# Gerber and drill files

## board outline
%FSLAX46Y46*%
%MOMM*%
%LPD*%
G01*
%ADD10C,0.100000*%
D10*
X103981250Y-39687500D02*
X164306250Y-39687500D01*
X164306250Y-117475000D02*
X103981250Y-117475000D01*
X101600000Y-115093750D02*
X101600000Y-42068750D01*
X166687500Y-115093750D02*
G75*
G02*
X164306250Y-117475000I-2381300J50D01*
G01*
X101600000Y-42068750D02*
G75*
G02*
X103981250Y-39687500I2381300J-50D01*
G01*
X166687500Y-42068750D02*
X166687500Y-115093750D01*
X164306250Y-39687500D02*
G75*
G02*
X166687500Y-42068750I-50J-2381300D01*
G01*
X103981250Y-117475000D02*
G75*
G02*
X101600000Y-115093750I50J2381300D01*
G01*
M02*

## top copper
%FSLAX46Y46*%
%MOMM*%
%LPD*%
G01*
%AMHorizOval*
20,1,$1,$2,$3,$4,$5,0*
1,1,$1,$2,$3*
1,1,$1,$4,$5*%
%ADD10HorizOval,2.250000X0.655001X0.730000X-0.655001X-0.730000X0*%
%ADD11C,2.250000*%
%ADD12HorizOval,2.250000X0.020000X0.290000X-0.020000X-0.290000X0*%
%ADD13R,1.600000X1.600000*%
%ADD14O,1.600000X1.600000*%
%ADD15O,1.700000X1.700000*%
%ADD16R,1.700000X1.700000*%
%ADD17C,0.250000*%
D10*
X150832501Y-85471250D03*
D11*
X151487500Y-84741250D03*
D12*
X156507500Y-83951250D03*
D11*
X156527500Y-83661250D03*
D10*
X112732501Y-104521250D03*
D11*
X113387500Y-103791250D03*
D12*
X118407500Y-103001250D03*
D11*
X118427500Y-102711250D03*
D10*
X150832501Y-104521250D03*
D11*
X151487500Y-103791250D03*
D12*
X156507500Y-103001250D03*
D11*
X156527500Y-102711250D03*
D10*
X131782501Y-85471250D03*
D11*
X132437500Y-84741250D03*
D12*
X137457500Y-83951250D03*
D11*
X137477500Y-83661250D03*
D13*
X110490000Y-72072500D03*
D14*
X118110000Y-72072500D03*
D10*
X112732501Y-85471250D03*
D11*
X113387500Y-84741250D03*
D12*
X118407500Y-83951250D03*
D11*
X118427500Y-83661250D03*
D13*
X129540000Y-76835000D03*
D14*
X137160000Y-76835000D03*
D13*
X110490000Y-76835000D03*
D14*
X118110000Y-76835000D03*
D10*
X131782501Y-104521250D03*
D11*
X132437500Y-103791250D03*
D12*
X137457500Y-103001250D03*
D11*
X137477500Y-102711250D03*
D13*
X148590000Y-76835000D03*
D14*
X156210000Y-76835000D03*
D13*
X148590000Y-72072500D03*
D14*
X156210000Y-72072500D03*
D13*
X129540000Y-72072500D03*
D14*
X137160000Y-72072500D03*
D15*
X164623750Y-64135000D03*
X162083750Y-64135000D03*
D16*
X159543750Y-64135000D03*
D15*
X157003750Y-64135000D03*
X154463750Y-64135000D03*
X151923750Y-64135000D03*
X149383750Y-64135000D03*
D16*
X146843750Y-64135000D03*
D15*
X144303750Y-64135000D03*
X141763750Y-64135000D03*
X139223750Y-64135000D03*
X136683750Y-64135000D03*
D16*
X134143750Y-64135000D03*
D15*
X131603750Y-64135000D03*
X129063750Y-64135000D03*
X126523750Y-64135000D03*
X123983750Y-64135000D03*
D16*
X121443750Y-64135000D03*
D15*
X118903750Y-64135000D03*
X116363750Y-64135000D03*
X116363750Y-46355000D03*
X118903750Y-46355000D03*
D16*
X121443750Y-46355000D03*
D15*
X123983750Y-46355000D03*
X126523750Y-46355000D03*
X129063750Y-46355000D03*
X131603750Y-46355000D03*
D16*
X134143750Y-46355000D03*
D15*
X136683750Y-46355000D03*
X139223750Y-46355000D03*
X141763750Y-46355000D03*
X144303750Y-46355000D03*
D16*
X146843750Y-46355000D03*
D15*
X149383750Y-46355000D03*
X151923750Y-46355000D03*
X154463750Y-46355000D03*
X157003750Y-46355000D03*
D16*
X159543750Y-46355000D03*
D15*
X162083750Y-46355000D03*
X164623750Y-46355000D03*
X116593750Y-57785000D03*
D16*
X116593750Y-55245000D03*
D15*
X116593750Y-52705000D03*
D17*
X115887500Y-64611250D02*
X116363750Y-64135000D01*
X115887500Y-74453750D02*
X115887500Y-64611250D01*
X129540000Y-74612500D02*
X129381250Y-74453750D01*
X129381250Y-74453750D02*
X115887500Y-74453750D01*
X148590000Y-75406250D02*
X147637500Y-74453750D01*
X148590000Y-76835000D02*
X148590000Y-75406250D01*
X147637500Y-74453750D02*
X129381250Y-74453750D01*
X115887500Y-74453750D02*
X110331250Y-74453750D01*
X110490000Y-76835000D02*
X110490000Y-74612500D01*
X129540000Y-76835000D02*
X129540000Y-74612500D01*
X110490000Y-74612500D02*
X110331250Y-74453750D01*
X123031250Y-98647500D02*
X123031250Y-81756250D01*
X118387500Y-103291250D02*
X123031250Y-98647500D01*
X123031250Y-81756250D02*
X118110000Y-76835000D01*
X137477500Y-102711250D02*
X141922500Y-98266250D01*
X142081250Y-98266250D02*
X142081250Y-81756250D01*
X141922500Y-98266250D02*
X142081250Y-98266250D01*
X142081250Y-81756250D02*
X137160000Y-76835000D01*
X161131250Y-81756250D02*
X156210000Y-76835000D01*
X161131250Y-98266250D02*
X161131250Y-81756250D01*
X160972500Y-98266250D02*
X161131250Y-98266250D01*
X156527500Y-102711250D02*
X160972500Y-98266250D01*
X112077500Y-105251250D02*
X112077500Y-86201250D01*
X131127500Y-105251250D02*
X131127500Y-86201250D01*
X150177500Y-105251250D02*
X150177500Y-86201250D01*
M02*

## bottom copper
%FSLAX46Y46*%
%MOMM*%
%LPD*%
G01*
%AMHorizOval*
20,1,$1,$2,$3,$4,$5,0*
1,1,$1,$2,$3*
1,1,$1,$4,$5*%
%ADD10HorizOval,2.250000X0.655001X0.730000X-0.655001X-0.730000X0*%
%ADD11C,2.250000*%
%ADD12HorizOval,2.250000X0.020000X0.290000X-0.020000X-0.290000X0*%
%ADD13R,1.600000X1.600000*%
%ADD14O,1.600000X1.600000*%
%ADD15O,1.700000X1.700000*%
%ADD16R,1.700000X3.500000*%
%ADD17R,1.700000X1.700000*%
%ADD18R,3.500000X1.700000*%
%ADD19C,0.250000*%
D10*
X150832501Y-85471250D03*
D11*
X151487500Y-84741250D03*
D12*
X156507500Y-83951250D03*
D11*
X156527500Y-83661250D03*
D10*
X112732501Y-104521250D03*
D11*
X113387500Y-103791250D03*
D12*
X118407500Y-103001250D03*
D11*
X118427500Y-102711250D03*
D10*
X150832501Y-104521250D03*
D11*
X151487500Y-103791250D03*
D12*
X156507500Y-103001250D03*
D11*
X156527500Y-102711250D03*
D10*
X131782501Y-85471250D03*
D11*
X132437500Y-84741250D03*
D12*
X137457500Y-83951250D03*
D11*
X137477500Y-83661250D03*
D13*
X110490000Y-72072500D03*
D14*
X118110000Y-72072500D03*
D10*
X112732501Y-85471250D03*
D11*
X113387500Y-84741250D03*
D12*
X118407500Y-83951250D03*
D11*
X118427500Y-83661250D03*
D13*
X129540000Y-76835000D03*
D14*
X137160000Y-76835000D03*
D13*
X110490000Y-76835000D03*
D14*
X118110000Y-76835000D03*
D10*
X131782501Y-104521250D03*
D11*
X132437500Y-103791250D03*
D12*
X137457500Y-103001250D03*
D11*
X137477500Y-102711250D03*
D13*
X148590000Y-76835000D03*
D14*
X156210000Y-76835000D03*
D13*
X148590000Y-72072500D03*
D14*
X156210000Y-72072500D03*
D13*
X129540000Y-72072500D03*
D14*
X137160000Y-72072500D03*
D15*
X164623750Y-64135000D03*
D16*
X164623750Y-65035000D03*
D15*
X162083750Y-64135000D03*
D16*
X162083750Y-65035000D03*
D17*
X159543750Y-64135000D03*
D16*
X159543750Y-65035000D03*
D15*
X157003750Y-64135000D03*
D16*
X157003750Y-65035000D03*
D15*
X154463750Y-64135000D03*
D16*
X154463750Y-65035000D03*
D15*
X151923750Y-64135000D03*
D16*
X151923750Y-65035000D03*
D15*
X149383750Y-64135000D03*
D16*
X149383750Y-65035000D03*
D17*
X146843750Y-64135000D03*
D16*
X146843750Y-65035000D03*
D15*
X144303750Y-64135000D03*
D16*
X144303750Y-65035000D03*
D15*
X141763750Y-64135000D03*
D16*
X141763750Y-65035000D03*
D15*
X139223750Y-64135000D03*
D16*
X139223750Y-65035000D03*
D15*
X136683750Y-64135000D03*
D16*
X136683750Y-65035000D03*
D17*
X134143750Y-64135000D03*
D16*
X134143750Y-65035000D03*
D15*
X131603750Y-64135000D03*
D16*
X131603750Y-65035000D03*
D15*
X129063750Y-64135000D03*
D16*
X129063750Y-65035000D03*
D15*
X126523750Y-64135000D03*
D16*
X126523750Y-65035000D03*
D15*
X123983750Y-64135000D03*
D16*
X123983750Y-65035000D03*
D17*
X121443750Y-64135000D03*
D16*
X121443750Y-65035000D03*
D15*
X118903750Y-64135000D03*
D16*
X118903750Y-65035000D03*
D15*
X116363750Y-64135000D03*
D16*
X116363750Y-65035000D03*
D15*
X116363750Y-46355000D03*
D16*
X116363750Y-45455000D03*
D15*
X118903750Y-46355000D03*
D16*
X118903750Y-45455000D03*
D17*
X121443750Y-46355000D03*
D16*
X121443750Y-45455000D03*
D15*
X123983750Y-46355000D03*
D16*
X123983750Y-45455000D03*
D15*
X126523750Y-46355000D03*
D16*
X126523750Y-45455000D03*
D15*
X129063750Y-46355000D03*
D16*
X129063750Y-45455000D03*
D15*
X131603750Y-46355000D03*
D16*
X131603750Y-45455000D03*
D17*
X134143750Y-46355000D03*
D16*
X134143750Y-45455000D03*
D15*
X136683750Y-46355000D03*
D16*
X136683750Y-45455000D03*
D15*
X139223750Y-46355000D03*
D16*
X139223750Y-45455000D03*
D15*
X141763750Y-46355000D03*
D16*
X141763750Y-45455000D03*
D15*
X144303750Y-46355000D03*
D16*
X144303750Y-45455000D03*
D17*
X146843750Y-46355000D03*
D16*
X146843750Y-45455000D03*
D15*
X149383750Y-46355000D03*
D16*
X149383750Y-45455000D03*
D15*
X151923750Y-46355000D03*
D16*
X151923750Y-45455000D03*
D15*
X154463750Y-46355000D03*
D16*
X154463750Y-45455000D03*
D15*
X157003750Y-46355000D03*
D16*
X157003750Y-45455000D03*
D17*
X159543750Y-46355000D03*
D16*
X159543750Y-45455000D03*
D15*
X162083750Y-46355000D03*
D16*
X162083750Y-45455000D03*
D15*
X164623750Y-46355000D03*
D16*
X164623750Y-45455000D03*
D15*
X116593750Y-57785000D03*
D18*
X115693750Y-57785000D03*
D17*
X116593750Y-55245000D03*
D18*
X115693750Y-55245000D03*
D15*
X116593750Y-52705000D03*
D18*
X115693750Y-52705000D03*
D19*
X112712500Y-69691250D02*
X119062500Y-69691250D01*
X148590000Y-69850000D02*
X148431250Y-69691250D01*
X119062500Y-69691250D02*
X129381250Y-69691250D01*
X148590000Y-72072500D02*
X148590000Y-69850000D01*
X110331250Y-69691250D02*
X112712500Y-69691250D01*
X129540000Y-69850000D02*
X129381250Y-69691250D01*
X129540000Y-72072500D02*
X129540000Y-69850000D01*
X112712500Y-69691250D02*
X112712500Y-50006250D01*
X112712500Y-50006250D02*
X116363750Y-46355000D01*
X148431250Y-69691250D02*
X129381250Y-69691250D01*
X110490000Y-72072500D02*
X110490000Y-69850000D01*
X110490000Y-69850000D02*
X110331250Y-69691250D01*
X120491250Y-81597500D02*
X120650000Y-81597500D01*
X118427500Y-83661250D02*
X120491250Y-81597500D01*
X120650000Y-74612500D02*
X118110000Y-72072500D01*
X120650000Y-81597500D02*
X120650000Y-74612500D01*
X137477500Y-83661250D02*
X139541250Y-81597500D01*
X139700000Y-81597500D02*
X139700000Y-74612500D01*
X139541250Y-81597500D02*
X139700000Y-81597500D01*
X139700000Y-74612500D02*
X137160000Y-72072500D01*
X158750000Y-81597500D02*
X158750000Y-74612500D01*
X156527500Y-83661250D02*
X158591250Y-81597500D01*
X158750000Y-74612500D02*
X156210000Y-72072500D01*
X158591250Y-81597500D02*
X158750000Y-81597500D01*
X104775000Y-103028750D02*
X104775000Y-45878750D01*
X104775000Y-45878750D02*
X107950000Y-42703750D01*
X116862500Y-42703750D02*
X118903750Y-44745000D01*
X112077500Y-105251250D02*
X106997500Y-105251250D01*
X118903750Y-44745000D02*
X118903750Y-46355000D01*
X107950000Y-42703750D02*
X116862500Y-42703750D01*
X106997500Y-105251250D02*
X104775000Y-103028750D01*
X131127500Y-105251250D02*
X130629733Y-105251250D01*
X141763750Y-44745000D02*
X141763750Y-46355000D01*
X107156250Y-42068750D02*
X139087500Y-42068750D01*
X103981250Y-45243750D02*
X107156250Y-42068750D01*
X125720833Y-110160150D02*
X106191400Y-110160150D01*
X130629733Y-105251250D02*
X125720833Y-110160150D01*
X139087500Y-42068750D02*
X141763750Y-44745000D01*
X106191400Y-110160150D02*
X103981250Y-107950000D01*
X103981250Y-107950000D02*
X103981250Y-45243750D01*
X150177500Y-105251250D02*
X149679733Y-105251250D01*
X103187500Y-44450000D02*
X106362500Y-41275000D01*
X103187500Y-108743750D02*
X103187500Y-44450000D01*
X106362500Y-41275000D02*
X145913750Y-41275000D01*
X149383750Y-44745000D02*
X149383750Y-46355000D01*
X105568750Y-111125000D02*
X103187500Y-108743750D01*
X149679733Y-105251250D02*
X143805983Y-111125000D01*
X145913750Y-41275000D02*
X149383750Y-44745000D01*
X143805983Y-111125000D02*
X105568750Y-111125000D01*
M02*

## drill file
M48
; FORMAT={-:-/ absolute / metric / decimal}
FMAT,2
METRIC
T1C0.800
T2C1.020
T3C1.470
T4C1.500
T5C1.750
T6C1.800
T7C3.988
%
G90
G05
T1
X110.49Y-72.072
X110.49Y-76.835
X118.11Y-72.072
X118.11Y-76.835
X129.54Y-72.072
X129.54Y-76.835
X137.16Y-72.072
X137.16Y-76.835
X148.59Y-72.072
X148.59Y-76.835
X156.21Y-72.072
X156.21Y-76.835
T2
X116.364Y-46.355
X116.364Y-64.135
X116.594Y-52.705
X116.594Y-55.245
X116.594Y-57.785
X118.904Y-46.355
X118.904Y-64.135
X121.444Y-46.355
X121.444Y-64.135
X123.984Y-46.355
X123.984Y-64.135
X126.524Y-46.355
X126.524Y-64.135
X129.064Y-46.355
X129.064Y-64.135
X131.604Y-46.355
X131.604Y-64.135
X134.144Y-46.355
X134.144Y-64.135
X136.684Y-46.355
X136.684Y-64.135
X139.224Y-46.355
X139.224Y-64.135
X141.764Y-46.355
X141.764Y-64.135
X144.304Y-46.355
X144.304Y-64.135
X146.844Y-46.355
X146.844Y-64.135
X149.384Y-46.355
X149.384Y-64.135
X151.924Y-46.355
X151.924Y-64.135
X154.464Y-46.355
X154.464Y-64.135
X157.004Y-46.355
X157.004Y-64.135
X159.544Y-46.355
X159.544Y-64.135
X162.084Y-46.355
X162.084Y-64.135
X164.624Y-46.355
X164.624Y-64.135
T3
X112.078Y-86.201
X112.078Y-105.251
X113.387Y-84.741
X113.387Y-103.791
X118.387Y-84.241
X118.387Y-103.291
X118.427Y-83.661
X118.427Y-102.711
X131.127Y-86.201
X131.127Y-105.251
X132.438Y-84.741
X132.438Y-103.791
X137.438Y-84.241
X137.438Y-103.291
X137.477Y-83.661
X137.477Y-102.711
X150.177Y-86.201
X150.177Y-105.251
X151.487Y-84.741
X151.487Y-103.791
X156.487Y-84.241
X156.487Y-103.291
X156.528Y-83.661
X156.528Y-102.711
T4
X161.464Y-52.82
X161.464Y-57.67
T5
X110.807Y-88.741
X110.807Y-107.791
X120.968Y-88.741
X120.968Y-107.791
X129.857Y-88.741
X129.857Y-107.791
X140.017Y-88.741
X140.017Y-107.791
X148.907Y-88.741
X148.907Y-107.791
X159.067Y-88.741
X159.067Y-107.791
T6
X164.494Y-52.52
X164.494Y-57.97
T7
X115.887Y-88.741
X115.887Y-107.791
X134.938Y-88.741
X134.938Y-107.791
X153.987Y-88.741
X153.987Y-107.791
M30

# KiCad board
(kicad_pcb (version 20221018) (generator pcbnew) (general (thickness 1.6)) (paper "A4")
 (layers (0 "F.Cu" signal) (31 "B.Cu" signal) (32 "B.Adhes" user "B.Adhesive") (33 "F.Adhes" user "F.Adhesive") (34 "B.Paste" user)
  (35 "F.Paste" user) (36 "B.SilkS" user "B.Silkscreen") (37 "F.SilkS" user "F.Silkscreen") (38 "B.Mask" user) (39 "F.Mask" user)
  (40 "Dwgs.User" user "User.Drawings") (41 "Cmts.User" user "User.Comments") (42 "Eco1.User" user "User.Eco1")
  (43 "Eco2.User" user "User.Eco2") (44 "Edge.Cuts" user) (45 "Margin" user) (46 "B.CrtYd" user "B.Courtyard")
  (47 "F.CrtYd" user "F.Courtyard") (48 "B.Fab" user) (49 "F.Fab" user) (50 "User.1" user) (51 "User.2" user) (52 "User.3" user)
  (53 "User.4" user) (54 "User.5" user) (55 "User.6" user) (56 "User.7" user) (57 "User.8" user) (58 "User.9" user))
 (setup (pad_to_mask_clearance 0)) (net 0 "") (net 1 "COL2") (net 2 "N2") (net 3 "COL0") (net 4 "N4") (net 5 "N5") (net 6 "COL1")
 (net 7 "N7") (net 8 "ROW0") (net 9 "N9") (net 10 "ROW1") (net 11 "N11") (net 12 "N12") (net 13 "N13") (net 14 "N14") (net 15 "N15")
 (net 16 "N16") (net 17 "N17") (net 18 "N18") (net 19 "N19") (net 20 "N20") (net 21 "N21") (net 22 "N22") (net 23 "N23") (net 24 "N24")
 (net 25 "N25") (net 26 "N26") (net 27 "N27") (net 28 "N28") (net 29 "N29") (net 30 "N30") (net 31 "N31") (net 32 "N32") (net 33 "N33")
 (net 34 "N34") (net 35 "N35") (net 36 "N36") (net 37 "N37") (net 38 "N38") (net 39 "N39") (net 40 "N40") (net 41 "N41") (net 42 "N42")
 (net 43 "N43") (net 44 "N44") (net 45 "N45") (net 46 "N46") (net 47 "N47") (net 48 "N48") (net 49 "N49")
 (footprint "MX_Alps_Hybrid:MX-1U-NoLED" (layer "F.Cu") (at 153.9875 88.74125)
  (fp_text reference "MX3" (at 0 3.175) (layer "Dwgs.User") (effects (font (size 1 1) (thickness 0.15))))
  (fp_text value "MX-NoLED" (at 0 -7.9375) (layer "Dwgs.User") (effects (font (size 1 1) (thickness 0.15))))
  (pad "" np_thru_hole circle (at -5.08 0 48.0996) (size 1.75 1.75) (drill 1.75) (layers "*.Cu" "*.Mask"))
  (pad "" np_thru_hole circle (at 0 0) (size 3.9878 3.9878) (drill 3.9878) (layers "*.Cu" "*.Mask"))
  (pad "" np_thru_hole circle (at 5.08 0 48.0996) (size 1.75 1.75) (drill 1.75) (layers "*.Cu" "*.Mask"))
  (pad "1" thru_hole oval (at -3.81 -2.54 48.0996) (size 4.211556 2.25) (drill 1.47 (offset 0.980778 0)) (layers "*.Cu" "B.Mask")
   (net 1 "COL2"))
  (pad "1" thru_hole circle (at -2.5 -4) (size 2.25 2.25) (drill 1.47) (layers "*.Cu" "B.Mask") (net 1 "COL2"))
  (pad "2" thru_hole oval (at 2.5 -4.5 86.0548) (size 2.831378 2.25) (drill 1.47 (offset 0.290689 0)) (layers "*.Cu" "B.Mask") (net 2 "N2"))
  (pad "2" thru_hole circle (at 2.54 -5.08) (size 2.25 2.25) (drill 1.47) (layers "*.Cu" "B.Mask") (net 2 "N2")))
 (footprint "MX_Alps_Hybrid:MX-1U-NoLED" (layer "F.Cu") (at 115.8875 107.79125)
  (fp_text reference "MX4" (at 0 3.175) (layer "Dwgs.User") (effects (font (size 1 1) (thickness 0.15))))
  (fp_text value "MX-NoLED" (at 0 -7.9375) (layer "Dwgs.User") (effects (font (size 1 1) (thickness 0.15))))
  (pad "" np_thru_hole circle (at -5.08 0 48.0996) (size 1.75 1.75) (drill 1.75) (layers "*.Cu" "*.Mask"))
  (pad "" np_thru_hole circle (at 0 0) (size 3.9878 3.9878) (drill 3.9878) (layers "*.Cu" "*.Mask"))
  (pad "" np_thru_hole circle (at 5.08 0 48.0996) (size 1.75 1.75) (drill 1.75) (layers "*.Cu" "*.Mask"))
  (pad "1" thru_hole oval (at -3.81 -2.54 48.0996) (size 4.211556 2.25) (drill 1.47 (offset 0.980778 0)) (layers "*.Cu" "B.Mask")
   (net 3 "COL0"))
  (pad "1" thru_hole circle (at -2.5 -4) (size 2.25 2.25) (drill 1.47) (layers "*.Cu" "B.Mask") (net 3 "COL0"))
  (pad "2" thru_hole oval (at 2.5 -4.5 86.0548) (size 2.831378 2.25) (drill 1.47 (offset 0.290689 0)) (layers "*.Cu" "B.Mask") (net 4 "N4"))
  (pad "2" thru_hole circle (at 2.54 -5.08) (size 2.25 2.25) (drill 1.47) (layers "*.Cu" "B.Mask") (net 4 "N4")))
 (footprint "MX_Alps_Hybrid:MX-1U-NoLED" (layer "F.Cu") (at 153.9875 107.79125)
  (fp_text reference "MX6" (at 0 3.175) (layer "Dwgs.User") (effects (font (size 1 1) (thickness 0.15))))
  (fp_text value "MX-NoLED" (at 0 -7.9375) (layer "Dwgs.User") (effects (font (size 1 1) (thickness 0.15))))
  (pad "" np_thru_hole circle (at -5.08 0 48.0996) (size 1.75 1.75) (drill 1.75) (layers "*.Cu" "*.Mask"))
  (pad "" np_thru_hole circle (at 0 0) (size 3.9878 3.9878) (drill 3.9878) (layers "*.Cu" "*.Mask"))
  (pad "" np_thru_hole circle (at 5.08 0 48.0996) (size 1.75 1.75) (drill 1.75) (layers "*.Cu" "*.Mask"))
  (pad "1" thru_hole oval (at -3.81 -2.54 48.0996) (size 4.211556 2.25) (drill 1.47 (offset 0.980778 0)) (layers "*.Cu" "B.Mask")
   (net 1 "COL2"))
  (pad "1" thru_hole circle (at -2.5 -4) (size 2.25 2.25) (drill 1.47) (layers "*.Cu" "B.Mask") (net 1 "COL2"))
  (pad "2" thru_hole oval (at 2.5 -4.5 86.0548) (size 2.831378 2.25) (drill 1.47 (offset 0.290689 0)) (layers "*.Cu" "B.Mask") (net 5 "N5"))
  (pad "2" thru_hole circle (at 2.54 -5.08) (size 2.25 2.25) (drill 1.47) (layers "*.Cu" "B.Mask") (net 5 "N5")))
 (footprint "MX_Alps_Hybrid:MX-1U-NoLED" (layer "F.Cu") (at 134.9375 88.74125)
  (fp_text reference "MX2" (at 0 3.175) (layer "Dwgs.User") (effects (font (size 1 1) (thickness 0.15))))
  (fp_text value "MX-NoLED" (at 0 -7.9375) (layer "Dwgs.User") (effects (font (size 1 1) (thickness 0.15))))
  (pad "" np_thru_hole circle (at -5.08 0 48.0996) (size 1.75 1.75) (drill 1.75) (layers "*.Cu" "*.Mask"))
  (pad "" np_thru_hole circle (at 0 0) (size 3.9878 3.9878) (drill 3.9878) (layers "*.Cu" "*.Mask"))
  (pad "" np_thru_hole circle (at 5.08 0 48.0996) (size 1.75 1.75) (drill 1.75) (layers "*.Cu" "*.Mask"))
  (pad "1" thru_hole oval (at -3.81 -2.54 48.0996) (size 4.211556 2.25) (drill 1.47 (offset 0.980778 0)) (layers "*.Cu" "B.Mask")
   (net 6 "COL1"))
  (pad "1" thru_hole circle (at -2.5 -4) (size 2.25 2.25) (drill 1.47) (layers "*.Cu" "B.Mask") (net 6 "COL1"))
  (pad "2" thru_hole oval (at 2.5 -4.5 86.0548) (size 2.831378 2.25) (drill 1.47 (offset 0.290689 0)) (layers "*.Cu" "B.Mask") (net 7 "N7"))
  (pad "2" thru_hole circle (at 2.54 -5.08) (size 2.25 2.25) (drill 1.47) (layers "*.Cu" "B.Mask") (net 7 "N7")))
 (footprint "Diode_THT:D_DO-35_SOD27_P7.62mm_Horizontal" (layer "F.Cu") (at 110.49 72.0725)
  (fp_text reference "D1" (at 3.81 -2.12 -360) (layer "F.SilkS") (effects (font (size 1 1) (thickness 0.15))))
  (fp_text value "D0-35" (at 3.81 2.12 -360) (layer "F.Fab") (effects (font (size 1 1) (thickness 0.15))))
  (pad "1" thru_hole rect (at 0 0) (size 1.6 1.6) (drill 0.8) (layers "*.Cu" "*.Mask") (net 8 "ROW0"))
  (pad "2" thru_hole oval (at 7.62 0) (size 1.6 1.6) (drill 0.8) (layers "*.Cu" "*.Mask") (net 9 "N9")))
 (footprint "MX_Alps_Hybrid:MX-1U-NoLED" (layer "F.Cu") (at 115.8875 88.74125)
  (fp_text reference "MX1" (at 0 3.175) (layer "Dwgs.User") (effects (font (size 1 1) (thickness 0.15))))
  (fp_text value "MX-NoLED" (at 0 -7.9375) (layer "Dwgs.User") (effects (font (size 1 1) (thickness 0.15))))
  (pad "" np_thru_hole circle (at -5.08 0 48.0996) (size 1.75 1.75) (drill 1.75) (layers "*.Cu" "*.Mask"))
  (pad "" np_thru_hole circle (at 0 0) (size 3.9878 3.9878) (drill 3.9878) (layers "*.Cu" "*.Mask"))
  (pad "" np_thru_hole circle (at 5.08 0 48.0996) (size 1.75 1.75) (drill 1.75) (layers "*.Cu" "*.Mask"))
  (pad "1" thru_hole oval (at -3.81 -2.54 48.0996) (size 4.211556 2.25) (drill 1.47 (offset 0.980778 0)) (layers "*.Cu" "B.Mask")
   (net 3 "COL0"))
  (pad "1" thru_hole circle (at -2.5 -4) (size 2.25 2.25) (drill 1.47) (layers "*.Cu" "B.Mask") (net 3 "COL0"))
  (pad "2" thru_hole oval (at 2.5 -4.5 86.0548) (size 2.831378 2.25) (drill 1.47 (offset 0.290689 0)) (layers "*.Cu" "B.Mask") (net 9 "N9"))
  (pad "2" thru_hole circle (at 2.54 -5.08) (size 2.25 2.25) (drill 1.47) (layers "*.Cu" "B.Mask") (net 9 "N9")))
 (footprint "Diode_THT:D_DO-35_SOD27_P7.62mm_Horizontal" (layer "F.Cu") (at 129.54 76.835)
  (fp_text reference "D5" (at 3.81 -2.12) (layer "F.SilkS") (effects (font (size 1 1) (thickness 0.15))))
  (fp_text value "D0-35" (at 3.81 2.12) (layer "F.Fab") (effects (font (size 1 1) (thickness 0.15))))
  (pad "1" thru_hole rect (at 0 0) (size 1.6 1.6) (drill 0.8) (layers "*.Cu" "*.Mask") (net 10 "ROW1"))
  (pad "2" thru_hole oval (at 7.62 0) (size 1.6 1.6) (drill 0.8) (layers "*.Cu" "*.Mask") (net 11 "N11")))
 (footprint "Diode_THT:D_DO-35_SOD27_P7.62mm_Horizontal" (layer "F.Cu") (at 110.49 76.835)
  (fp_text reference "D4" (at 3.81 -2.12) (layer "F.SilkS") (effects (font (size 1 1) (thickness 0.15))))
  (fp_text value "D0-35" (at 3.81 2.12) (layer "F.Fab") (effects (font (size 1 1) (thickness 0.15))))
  (pad "1" thru_hole rect (at 0 0) (size 1.6 1.6) (drill 0.8) (layers "*.Cu" "*.Mask") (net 10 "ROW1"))
  (pad "2" thru_hole oval (at 7.62 0) (size 1.6 1.6) (drill 0.8) (layers "*.Cu" "*.Mask") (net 4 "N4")))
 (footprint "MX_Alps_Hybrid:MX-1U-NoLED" (layer "F.Cu") (at 134.9375 107.79125)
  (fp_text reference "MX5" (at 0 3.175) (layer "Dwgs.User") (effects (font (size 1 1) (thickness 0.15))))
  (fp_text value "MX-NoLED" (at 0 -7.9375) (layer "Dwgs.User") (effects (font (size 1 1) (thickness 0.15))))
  (pad "" np_thru_hole circle (at -5.08 0 48.0996) (size 1.75 1.75) (drill 1.75) (layers "*.Cu" "*.Mask"))
  (pad "" np_thru_hole circle (at 0 0) (size 3.9878 3.9878) (drill 3.9878) (layers "*.Cu" "*.Mask"))
  (pad "" np_thru_hole circle (at 5.08 0 48.0996) (size 1.75 1.75) (drill 1.75) (layers "*.Cu" "*.Mask"))
  (pad "1" thru_hole oval (at -3.81 -2.54 48.0996) (size 4.211556 2.25) (drill 1.47 (offset 0.980778 0)) (layers "*.Cu" "B.Mask")
   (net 6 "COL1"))
  (pad "1" thru_hole circle (at -2.5 -4) (size 2.25 2.25) (drill 1.47) (layers "*.Cu" "B.Mask") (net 6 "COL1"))
  (pad "2" thru_hole oval (at 2.5 -4.5 86.0548) (size 2.831378 2.25) (drill 1.47 (offset 0.290689 0)) (layers "*.Cu" "B.Mask")
   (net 11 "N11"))
  (pad "2" thru_hole circle (at 2.54 -5.08) (size 2.25 2.25) (drill 1.47) (layers "*.Cu" "B.Mask") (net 11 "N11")))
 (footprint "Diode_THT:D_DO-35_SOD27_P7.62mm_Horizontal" (layer "F.Cu") (at 148.59 76.835)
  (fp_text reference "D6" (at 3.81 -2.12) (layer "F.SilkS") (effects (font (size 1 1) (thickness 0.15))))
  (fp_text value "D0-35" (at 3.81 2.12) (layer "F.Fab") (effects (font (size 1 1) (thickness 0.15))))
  (pad "1" thru_hole rect (at 0 0) (size 1.6 1.6) (drill 0.8) (layers "*.Cu" "*.Mask") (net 10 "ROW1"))
  (pad "2" thru_hole oval (at 7.62 0) (size 1.6 1.6) (drill 0.8) (layers "*.Cu" "*.Mask") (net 5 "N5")))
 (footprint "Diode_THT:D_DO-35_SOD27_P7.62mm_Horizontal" (layer "F.Cu") (at 148.59 72.0725)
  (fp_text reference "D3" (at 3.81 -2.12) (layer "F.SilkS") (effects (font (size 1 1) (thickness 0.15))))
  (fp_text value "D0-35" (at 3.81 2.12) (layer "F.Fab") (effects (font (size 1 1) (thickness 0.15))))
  (pad "1" thru_hole rect (at 0 0) (size 1.6 1.6) (drill 0.8) (layers "*.Cu" "*.Mask") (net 8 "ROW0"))
  (pad "2" thru_hole oval (at 7.62 0) (size 1.6 1.6) (drill 0.8) (layers "*.Cu" "*.Mask") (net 2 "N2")))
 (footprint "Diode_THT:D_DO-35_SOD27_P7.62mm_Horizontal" (layer "F.Cu") (at 129.54 72.0725)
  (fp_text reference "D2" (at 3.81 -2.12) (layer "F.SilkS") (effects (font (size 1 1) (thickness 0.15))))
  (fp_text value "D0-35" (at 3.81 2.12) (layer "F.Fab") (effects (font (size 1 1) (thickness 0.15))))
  (pad "1" thru_hole rect (at 0 0) (size 1.6 1.6) (drill 0.8) (layers "*.Cu" "*.Mask") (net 8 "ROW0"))
  (pad "2" thru_hole oval (at 7.62 0) (size 1.6 1.6) (drill 0.8) (layers "*.Cu" "*.Mask") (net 7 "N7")))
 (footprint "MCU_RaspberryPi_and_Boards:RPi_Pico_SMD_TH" (layer "B.Cu") (at 140.49375 55.245 90)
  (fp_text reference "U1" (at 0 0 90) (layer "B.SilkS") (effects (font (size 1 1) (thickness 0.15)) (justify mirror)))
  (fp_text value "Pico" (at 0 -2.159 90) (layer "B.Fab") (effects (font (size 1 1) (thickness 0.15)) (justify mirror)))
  (pad "" np_thru_hole oval (at -2.725 24 90) (size 1.8 1.8) (drill 1.8) (layers "*.Cu" "*.Mask"))
  (pad "" np_thru_hole oval (at -2.425 20.97 90) (size 1.5 1.5) (drill 1.5) (layers "*.Cu" "*.Mask"))
  (pad "" np_thru_hole oval (at 2.425 20.97 90) (size 1.5 1.5) (drill 1.5) (layers "*.Cu" "*.Mask"))
  (pad "" np_thru_hole oval (at 2.725 24 90) (size 1.8 1.8) (drill 1.8) (layers "*.Cu" "*.Mask"))
  (pad "1" thru_hole oval (at -8.89 24.13 90) (size 1.7 1.7) (drill 1.02) (layers "*.Cu" "*.Mask") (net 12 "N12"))
  (pad "1" smd rect (at -8.89 24.13 90) (size 3.5 1.7) (drill (offset -0.9 0)) (layers "B.Cu" "B.Mask") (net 12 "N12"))
  (pad "2" thru_hole oval (at -8.89 21.59 90) (size 1.7 1.7) (drill 1.02) (layers "*.Cu" "*.Mask") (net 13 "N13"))
  (pad "2" smd rect (at -8.89 21.59 90) (size 3.5 1.7) (drill (offset -0.9 0)) (layers "B.Cu" "B.Mask") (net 13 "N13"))
  (pad "3" thru_hole rect (at -8.89 19.05 90) (size 1.7 1.7) (drill 1.02) (layers "*.Cu" "*.Mask") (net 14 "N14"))
  (pad "3" smd rect (at -8.89 19.05 90) (size 3.5 1.7) (drill (offset -0.9 0)) (layers "B.Cu" "B.Mask") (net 14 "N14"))
  (pad "4" thru_hole oval (at -8.89 16.51 90) (size 1.7 1.7) (drill 1.02) (layers "*.Cu" "*.Mask") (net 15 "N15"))
  (pad "4" smd rect (at -8.89 16.51 90) (size 3.5 1.7) (drill (offset -0.9 0)) (layers "B.Cu" "B.Mask") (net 15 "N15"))
  (pad "5" thru_hole oval (at -8.89 13.97 90) (size 1.7 1.7) (drill 1.02) (layers "*.Cu" "*.Mask") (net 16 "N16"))
  (pad "5" smd rect (at -8.89 13.97 90) (size 3.5 1.7) (drill (offset -0.9 0)) (layers "B.Cu" "B.Mask") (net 16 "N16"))
  (pad "6" thru_hole oval (at -8.89 11.43 90) (size 1.7 1.7) (drill 1.02) (layers "*.Cu" "*.Mask") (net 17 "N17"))
  (pad "6" smd rect (at -8.89 11.43 90) (size 3.5 1.7) (drill (offset -0.9 0)) (layers "B.Cu" "B.Mask") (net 17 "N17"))
  (pad "7" thru_hole oval (at -8.89 8.89 90) (size 1.7 1.7) (drill 1.02) (layers "*.Cu" "*.Mask") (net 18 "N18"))
  (pad "7" smd rect (at -8.89 8.89 90) (size 3.5 1.7) (drill (offset -0.9 0)) (layers "B.Cu" "B.Mask") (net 18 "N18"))
  (pad "8" thru_hole rect (at -8.89 6.35 90) (size 1.7 1.7) (drill 1.02) (layers "*.Cu" "*.Mask") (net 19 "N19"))
  (pad "8" smd rect (at -8.89 6.35 90) (size 3.5 1.7) (drill (offset -0.9 0)) (layers "B.Cu" "B.Mask") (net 19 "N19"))
  (pad "9" thru_hole oval (at -8.89 3.81 90) (size 1.7 1.7) (drill 1.02) (layers "*.Cu" "*.Mask") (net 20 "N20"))
  (pad "9" smd rect (at -8.89 3.81 90) (size 3.5 1.7) (drill (offset -0.9 0)) (layers "B.Cu" "B.Mask") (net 20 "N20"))
  (pad "10" thru_hole oval (at -8.89 1.27 90) (size 1.7 1.7) (drill 1.02) (layers "*.Cu" "*.Mask") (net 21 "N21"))
  (pad "10" smd rect (at -8.89 1.27 90) (size 3.5 1.7) (drill (offset -0.9 0)) (layers "B.Cu" "B.Mask") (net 21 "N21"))
  (pad "11" thru_hole oval (at -8.89 -1.27 90) (size 1.7 1.7) (drill 1.02) (layers "*.Cu" "*.Mask") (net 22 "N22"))
  (pad "11" smd rect (at -8.89 -1.27 90) (size 3.5 1.7) (drill (offset -0.9 0)) (layers "B.Cu" "B.Mask") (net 22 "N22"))
  (pad "12" thru_hole oval (at -8.89 -3.81 90) (size 1.7 1.7) (drill 1.02) (layers "*.Cu" "*.Mask") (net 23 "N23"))
  (pad "12" smd rect (at -8.89 -3.81 90) (size 3.5 1.7) (drill (offset -0.9 0)) (layers "B.Cu" "B.Mask") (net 23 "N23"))
  (pad "13" thru_hole rect (at -8.89 -6.35 90) (size 1.7 1.7) (drill 1.02) (layers "*.Cu" "*.Mask") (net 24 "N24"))
  (pad "13" smd rect (at -8.89 -6.35 90) (size 3.5 1.7) (drill (offset -0.9 0)) (layers "B.Cu" "B.Mask") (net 24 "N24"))
  (pad "14" thru_hole oval (at -8.89 -8.89 90) (size 1.7 1.7) (drill 1.02) (layers "*.Cu" "*.Mask") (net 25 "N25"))
  (pad "14" smd rect (at -8.89 -8.89 90) (size 3.5 1.7) (drill (offset -0.9 0)) (layers "B.Cu" "B.Mask") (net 25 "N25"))
  (pad "15" thru_hole oval (at -8.89 -11.43 90) (size 1.7 1.7) (drill 1.02) (layers "*.Cu" "*.Mask") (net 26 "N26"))
  (pad "15" smd rect (at -8.89 -11.43 90) (size 3.5 1.7) (drill (offset -0.9 0)) (layers "B.Cu" "B.Mask") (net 26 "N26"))
  (pad "16" thru_hole oval (at -8.89 -13.97 90) (size 1.7 1.7) (drill 1.02) (layers "*.Cu" "*.Mask") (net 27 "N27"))
  (pad "16" smd rect (at -8.89 -13.97 90) (size 3.5 1.7) (drill (offset -0.9 0)) (layers "B.Cu" "B.Mask") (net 27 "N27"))
  (pad "17" thru_hole oval (at -8.89 -16.51 90) (size 1.7 1.7) (drill 1.02) (layers "*.Cu" "*.Mask") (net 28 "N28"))
  (pad "17" smd rect (at -8.89 -16.51 90) (size 3.5 1.7) (drill (offset -0.9 0)) (layers "B.Cu" "B.Mask") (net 28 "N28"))
  (pad "18" thru_hole rect (at -8.89 -19.05 90) (size 1.7 1.7) (drill 1.02) (layers "*.Cu" "*.Mask") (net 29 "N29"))
  (pad "18" smd rect (at -8.89 -19.05 90) (size 3.5 1.7) (drill (offset -0.9 0)) (layers "B.Cu" "B.Mask") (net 29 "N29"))
  (pad "19" thru_hole oval (at -8.89 -21.59 90) (size 1.7 1.7) (drill 1.02) (layers "*.Cu" "*.Mask") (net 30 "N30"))
  (pad "19" smd rect (at -8.89 -21.59 90) (size 3.5 1.7) (drill (offset -0.9 0)) (layers "B.Cu" "B.Mask") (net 30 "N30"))
  (pad "20" thru_hole oval (at -8.89 -24.13 90) (size 1.7 1.7) (drill 1.02) (layers "*.Cu" "*.Mask") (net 10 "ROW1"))
  (pad "20" smd rect (at -8.89 -24.13 90) (size 3.5 1.7) (drill (offset -0.9 0)) (layers "B.Cu" "B.Mask") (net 10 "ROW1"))
  (pad "21" thru_hole oval (at 8.89 -24.13 90) (size 1.7 1.7) (drill 1.02) (layers "*.Cu" "*.Mask") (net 8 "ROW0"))
  (pad "21" smd rect (at 8.89 -24.13 90) (size 3.5 1.7) (drill (offset 0.9 0)) (layers "B.Cu" "B.Mask") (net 8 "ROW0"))
  (pad "22" thru_hole oval (at 8.89 -21.59 90) (size 1.7 1.7) (drill 1.02) (layers "*.Cu" "*.Mask") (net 3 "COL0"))
  (pad "22" smd rect (at 8.89 -21.59 90) (size 3.5 1.7) (drill (offset 0.9 0)) (layers "B.Cu" "B.Mask") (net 3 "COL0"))
  (pad "23" thru_hole rect (at 8.89 -19.05 90) (size 1.7 1.7) (drill 1.02) (layers "*.Cu" "*.Mask") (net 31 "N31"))
  (pad "23" smd rect (at 8.89 -19.05 90) (size 3.5 1.7) (drill (offset 0.9 0)) (layers "B.Cu" "B.Mask") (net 31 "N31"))
  (pad "24" thru_hole oval (at 8.89 -16.51 90) (size 1.7 1.7) (drill 1.02) (layers "*.Cu" "*.Mask") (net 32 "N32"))
  (pad "24" smd rect (at 8.89 -16.51 90) (size 3.5 1.7) (drill (offset 0.9 0)) (layers "B.Cu" "B.Mask") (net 32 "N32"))
  (pad "25" thru_hole oval (at 8.89 -13.97 90) (size 1.7 1.7) (drill 1.02) (layers "*.Cu" "*.Mask") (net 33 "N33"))
  (pad "25" smd rect (at 8.89 -13.97 90) (size 3.5 1.7) (drill (offset 0.9 0)) (layers "B.Cu" "B.Mask") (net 33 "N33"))
  (pad "26" thru_hole oval (at 8.89 -11.43 90) (size 1.7 1.7) (drill 1.02) (layers "*.Cu" "*.Mask") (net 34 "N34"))
  (pad "26" smd rect (at 8.89 -11.43 90) (size 3.5 1.7) (drill (offset 0.9 0)) (layers "B.Cu" "B.Mask") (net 34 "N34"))
  (pad "27" thru_hole oval (at 8.89 -8.89 90) (size 1.7 1.7) (drill 1.02) (layers "*.Cu" "*.Mask") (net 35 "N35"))
  (pad "27" smd rect (at 8.89 -8.89 90) (size 3.5 1.7) (drill (offset 0.9 0)) (layers "B.Cu" "B.Mask") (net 35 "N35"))
  (pad "28" thru_hole rect (at 8.89 -6.35 90) (size 1.7 1.7) (drill 1.02) (layers "*.Cu" "*.Mask") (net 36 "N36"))
  (pad "28" smd rect (at 8.89 -6.35 90) (size 3.5 1.7) (drill (offset 0.9 0)) (layers "B.Cu" "B.Mask") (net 36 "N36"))
  (pad "29" thru_hole oval (at 8.89 -3.81 90) (size 1.7 1.7) (drill 1.02) (layers "*.Cu" "*.Mask") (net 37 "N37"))
  (pad "29" smd rect (at 8.89 -3.81 90) (size 3.5 1.7) (drill (offset 0.9 0)) (layers "B.Cu" "B.Mask") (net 37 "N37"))
  (pad "30" thru_hole oval (at 8.89 -1.27 90) (size 1.7 1.7) (drill 1.02) (layers "*.Cu" "*.Mask") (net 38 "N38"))
  (pad "30" smd rect (at 8.89 -1.27 90) (size 3.5 1.7) (drill (offset 0.9 0)) (layers "B.Cu" "B.Mask") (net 38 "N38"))
  (pad "31" thru_hole oval (at 8.89 1.27 90) (size 1.7 1.7) (drill 1.02) (layers "*.Cu" "*.Mask") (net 6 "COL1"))
  (pad "31" smd rect (at 8.89 1.27 90) (size 3.5 1.7) (drill (offset 0.9 0)) (layers "B.Cu" "B.Mask") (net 6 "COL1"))
  (pad "32" thru_hole oval (at 8.89 3.81 90) (size 1.7 1.7) (drill 1.02) (layers "*.Cu" "*.Mask") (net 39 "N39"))
  (pad "32" smd rect (at 8.89 3.81 90) (size 3.5 1.7) (drill (offset 0.9 0)) (layers "B.Cu" "B.Mask") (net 39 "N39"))
  (pad "33" thru_hole rect (at 8.89 6.35 90) (size 1.7 1.7) (drill 1.02) (layers "*.Cu" "*.Mask") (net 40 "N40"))
  (pad "33" smd rect (at 8.89 6.35 90) (size 3.5 1.7) (drill (offset 0.9 0)) (layers "B.Cu" "B.Mask") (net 40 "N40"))
  (pad "34" thru_hole oval (at 8.89 8.89 90) (size 1.7 1.7) (drill 1.02) (layers "*.Cu" "*.Mask") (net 1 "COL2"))
  (pad "34" smd rect (at 8.89 8.89 90) (size 3.5 1.7) (drill (offset 0.9 0)) (layers "B.Cu" "B.Mask") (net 1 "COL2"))
  (pad "35" thru_hole oval (at 8.89 11.43 90) (size 1.7 1.7) (drill 1.02) (layers "*.Cu" "*.Mask") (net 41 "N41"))
  (pad "35" smd rect (at 8.89 11.43 90) (size 3.5 1.7) (drill (offset 0.9 0)) (layers "B.Cu" "B.Mask") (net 41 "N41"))
  (pad "36" thru_hole oval (at 8.89 13.97 90) (size 1.7 1.7) (drill 1.02) (layers "*.Cu" "*.Mask") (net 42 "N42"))
  (pad "36" smd rect (at 8.89 13.97 90) (size 3.5 1.7) (drill (offset 0.9 0)) (layers "B.Cu" "B.Mask") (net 42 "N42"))
  (pad "37" thru_hole oval (at 8.89 16.51 90) (size 1.7 1.7) (drill 1.02) (layers "*.Cu" "*.Mask") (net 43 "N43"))
  (pad "37" smd rect (at 8.89 16.51 90) (size 3.5 1.7) (drill (offset 0.9 0)) (layers "B.Cu" "B.Mask") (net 43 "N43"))
  (pad "38" thru_hole rect (at 8.89 19.05 90) (size 1.7 1.7) (drill 1.02) (layers "*.Cu" "*.Mask") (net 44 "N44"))
  (pad "38" smd rect (at 8.89 19.05 90) (size 3.5 1.7) (drill (offset 0.9 0)) (layers "B.Cu" "B.Mask") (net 44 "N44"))
  (pad "39" thru_hole oval (at 8.89 21.59 90) (size 1.7 1.7) (drill 1.02) (layers "*.Cu" "*.Mask") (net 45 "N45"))
  (pad "39" smd rect (at 8.89 21.59 90) (size 3.5 1.7) (drill (offset 0.9 0)) (layers "B.Cu" "B.Mask") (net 45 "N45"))
  (pad "40" thru_hole oval (at 8.89 24.13 90) (size 1.7 1.7) (drill 1.02) (layers "*.Cu" "*.Mask") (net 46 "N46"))
  (pad "40" smd rect (at 8.89 24.13 90) (size 3.5 1.7) (drill (offset 0.9 0)) (layers "B.Cu" "B.Mask") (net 46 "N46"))
  (pad "41" thru_hole oval (at -2.54 -23.9 90) (size 1.7 1.7) (drill 1.02) (layers "*.Cu" "*.Mask") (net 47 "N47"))
  (pad "41" smd rect (at -2.54 -23.9) (size 3.5 1.7) (drill (offset -0.9 0)) (layers "B.Cu" "B.Mask") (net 47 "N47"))
  (pad "42" thru_hole rect (at 0 -23.9 90) (size 1.7 1.7) (drill 1.02) (layers "*.Cu" "*.Mask") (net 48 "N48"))
  (pad "42" smd rect (at 0 -23.9) (size 3.5 1.7) (drill (offset -0.9 0)) (layers "B.Cu" "B.Mask") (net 48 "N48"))
  (pad "43" thru_hole oval (at 2.54 -23.9 90) (size 1.7 1.7) (drill 1.02) (layers "*.Cu" "*.Mask") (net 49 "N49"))
  (pad "43" smd rect (at 2.54 -23.9) (size 3.5 1.7) (drill (offset -0.9 0)) (layers "B.Cu" "B.Mask") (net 49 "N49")))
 (gr_line (start 103.98125 39.6875) (end 164.30625 39.6875) (stroke (width 0.1) (type default)) (layer "Edge.Cuts"))
 (gr_line (start 164.30625 117.475) (end 103.98125 117.475) (stroke (width 0.1) (type default)) (layer "Edge.Cuts"))
 (gr_line (start 101.6 115.09375) (end 101.6 42.06875) (stroke (width 0.1) (type default)) (layer "Edge.Cuts"))
 (gr_arc (start 166.6875 115.09375) (mid 165.990048 116.777548) (end 164.30625 117.475) (stroke (width 0.1) (type default))
  (layer "Edge.Cuts"))
 (gr_arc (start 101.6 42.06875) (mid 102.297452 40.384952) (end 103.98125 39.6875) (stroke (width 0.1) (type default)) (layer "Edge.Cuts"))
 (gr_line (start 166.6875 42.06875) (end 166.6875 115.09375) (stroke (width 0.1) (type default)) (layer "Edge.Cuts"))
 (gr_arc (start 164.30625 39.6875) (mid 165.990048 40.384952) (end 166.6875 42.06875) (stroke (width 0.1) (type default))
  (layer "Edge.Cuts"))
 (gr_arc (start 103.98125 117.475) (mid 102.297452 116.777548) (end 101.6 115.09375) (stroke (width 0.1) (type default)) (layer "Edge.Cuts"))
 (segment (start 112.7125 69.69125) (end 119.0625 69.69125) (width 0.25) (layer "B.Cu") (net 8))
 (segment (start 148.59 69.85) (end 148.43125 69.69125) (width 0.25) (layer "B.Cu") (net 8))
 (segment (start 119.0625 69.69125) (end 129.38125 69.69125) (width 0.25) (layer "B.Cu") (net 8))
 (segment (start 148.59 72.0725) (end 148.59 69.85) (width 0.25) (layer "B.Cu") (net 8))
 (segment (start 110.33125 69.69125) (end 112.7125 69.69125) (width 0.25) (layer "B.Cu") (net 8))
 (segment (start 129.54 69.85) (end 129.38125 69.69125) (width 0.25) (layer "B.Cu") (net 8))
 (segment (start 129.54 72.0725) (end 129.54 69.85) (width 0.25) (layer "B.Cu") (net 8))
 (segment (start 112.7125 69.69125) (end 112.7125 50.00625) (width 0.25) (layer "B.Cu") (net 8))
 (segment (start 112.7125 50.00625) (end 116.36375 46.355) (width 0.25) (layer "B.Cu") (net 8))
 (segment (start 148.43125 69.69125) (end 129.38125 69.69125) (width 0.25) (layer "B.Cu") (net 8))
 (segment (start 110.49 72.0725) (end 110.49 69.85) (width 0.25) (layer "B.Cu") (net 8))
 (segment (start 110.49 69.85) (end 110.33125 69.69125) (width 0.25) (layer "B.Cu") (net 8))
 (segment (start 120.49125 81.5975) (end 120.65 81.5975) (width 0.25) (layer "B.Cu") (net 9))
 (segment (start 118.4275 83.66125) (end 120.49125 81.5975) (width 0.25) (layer "B.Cu") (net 9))
 (segment (start 120.65 74.6125) (end 118.11 72.0725) (width 0.25) (layer "B.Cu") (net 9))
 (segment (start 120.65 81.5975) (end 120.65 74.6125) (width 0.25) (layer "B.Cu") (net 9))
 (segment (start 137.4775 83.66125) (end 139.54125 81.5975) (width 0.25) (layer "B.Cu") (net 7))
 (segment (start 139.7 81.5975) (end 139.7 74.6125) (width 0.25) (layer "B.Cu") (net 7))
 (segment (start 139.54125 81.5975) (end 139.7 81.5975) (width 0.25) (layer "B.Cu") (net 7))
 (segment (start 139.7 74.6125) (end 137.16 72.0725) (width 0.25) (layer "B.Cu") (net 7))
 (segment (start 158.75 81.5975) (end 158.75 74.6125) (width 0.25) (layer "B.Cu") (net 2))
 (segment (start 156.5275 83.66125) (end 158.59125 81.5975) (width 0.25) (layer "B.Cu") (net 2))
 (segment (start 158.75 74.6125) (end 156.21 72.0725) (width 0.25) (layer "B.Cu") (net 2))
 (segment (start 158.59125 81.5975) (end 158.75 81.5975) (width 0.25) (layer "B.Cu") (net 2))
 (segment (start 115.8875 64.61125) (end 116.36375 64.135) (width 0.25) (layer "F.Cu") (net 10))
 (segment (start 115.8875 74.45375) (end 115.8875 64.61125) (width 0.25) (layer "F.Cu") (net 10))
 (segment (start 129.54 74.6125) (end 129.38125 74.45375) (width 0.25) (layer "F.Cu") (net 10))
 (segment (start 129.38125 74.45375) (end 115.8875 74.45375) (width 0.25) (layer "F.Cu") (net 10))
 (segment (start 148.59 75.40625) (end 147.6375 74.45375) (width 0.25) (layer "F.Cu") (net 10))
 (segment (start 148.59 76.835) (end 148.59 75.40625) (width 0.25) (layer "F.Cu") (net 10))
 (segment (start 147.6375 74.45375) (end 129.38125 74.45375) (width 0.25) (layer "F.Cu") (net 10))
 (segment (start 115.8875 74.45375) (end 110.33125 74.45375) (width 0.25) (layer "F.Cu") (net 10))
 (segment (start 110.49 76.835) (end 110.49 74.6125) (width 0.25) (layer "F.Cu") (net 10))
 (segment (start 129.54 76.835) (end 129.54 74.6125) (width 0.25) (layer "F.Cu") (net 10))
 (segment (start 110.49 74.6125) (end 110.33125 74.45375) (width 0.25) (layer "F.Cu") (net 10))
 (segment (start 123.03125 98.6475) (end 123.03125 81.75625) (width 0.25) (layer "F.Cu") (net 4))
 (segment (start 118.3875 103.29125) (end 123.03125 98.6475) (width 0.25) (layer "F.Cu") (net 4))
 (segment (start 123.03125 81.75625) (end 118.11 76.835) (width 0.25) (layer "F.Cu") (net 4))
 (segment (start 137.4775 102.71125) (end 141.9225 98.26625) (width 0.25) (layer "F.Cu") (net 11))
 (segment (start 142.08125 98.26625) (end 142.08125 81.75625) (width 0.25) (layer "F.Cu") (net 11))
 (segment (start 141.9225 98.26625) (end 142.08125 98.26625) (width 0.25) (layer "F.Cu") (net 11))
 (segment (start 142.08125 81.75625) (end 137.16 76.835) (width 0.25) (layer "F.Cu") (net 11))
 (segment (start 161.13125 81.75625) (end 156.21 76.835) (width 0.25) (layer "F.Cu") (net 5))
 (segment (start 161.13125 98.26625) (end 161.13125 81.75625) (width 0.25) (layer "F.Cu") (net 5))
 (segment (start 160.9725 98.26625) (end 161.13125 98.26625) (width 0.25) (layer "F.Cu") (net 5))
 (segment (start 156.5275 102.71125) (end 160.9725 98.26625) (width 0.25) (layer "F.Cu") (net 5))
 (segment (start 112.0775 105.25125) (end 112.0775 86.20125) (width 0.25) (layer "F.Cu") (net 3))
 (segment (start 104.775 103.02875) (end 104.775 45.87875) (width 0.25) (layer "B.Cu") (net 3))
 (segment (start 104.775 45.87875) (end 107.95 42.70375) (width 0.25) (layer "B.Cu") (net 3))
 (segment (start 116.8625 42.70375) (end 118.90375 44.745) (width 0.25) (layer "B.Cu") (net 3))
 (segment (start 112.0775 105.25125) (end 106.9975 105.25125) (width 0.25) (layer "B.Cu") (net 3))
 (segment (start 118.90375 44.745) (end 118.90375 46.355) (width 0.25) (layer "B.Cu") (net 3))
 (segment (start 107.95 42.70375) (end 116.8625 42.70375) (width 0.25) (layer "B.Cu") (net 3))
 (segment (start 106.9975 105.25125) (end 104.775 103.02875) (width 0.25) (layer "B.Cu") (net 3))
 (segment (start 131.1275 105.25125) (end 131.1275 86.20125) (width 0.25) (layer "F.Cu") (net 6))
 (segment (start 131.1275 105.25125) (end 130.629733 105.25125) (width 0.25) (layer "B.Cu") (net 6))
 (segment (start 141.76375 44.745) (end 141.76375 46.355) (width 0.25) (layer "B.Cu") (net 6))
 (segment (start 107.15625 42.06875) (end 139.0875 42.06875) (width 0.25) (layer "B.Cu") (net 6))
 (segment (start 103.98125 45.24375) (end 107.15625 42.06875) (width 0.25) (layer "B.Cu") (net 6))
 (segment (start 125.720833 110.16015) (end 106.1914 110.16015) (width 0.25) (layer "B.Cu") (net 6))
 (segment (start 130.629733 105.25125) (end 125.720833 110.16015) (width 0.25) (layer "B.Cu") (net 6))
 (segment (start 139.0875 42.06875) (end 141.76375 44.745) (width 0.25) (layer "B.Cu") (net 6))
 (segment (start 106.1914 110.16015) (end 103.98125 107.95) (width 0.25) (layer "B.Cu") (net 6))
 (segment (start 103.98125 107.95) (end 103.98125 45.24375) (width 0.25) (layer "B.Cu") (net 6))
 (segment (start 150.1775 105.25125) (end 150.1775 86.20125) (width 0.25) (layer "F.Cu") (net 1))
 (segment (start 150.1775 105.25125) (end 149.679733 105.25125) (width 0.25) (layer "B.Cu") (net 1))
 (segment (start 103.1875 44.45) (end 106.3625 41.275) (width 0.25) (layer "B.Cu") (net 1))
 (segment (start 103.1875 108.74375) (end 103.1875 44.45) (width 0.25) (layer "B.Cu") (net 1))
 (segment (start 106.3625 41.275) (end 145.91375 41.275) (width 0.25) (layer "B.Cu") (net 1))
 (segment (start 149.38375 44.745) (end 149.38375 46.355) (width 0.25) (layer "B.Cu") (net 1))
 (segment (start 105.56875 111.125) (end 103.1875 108.74375) (width 0.25) (layer "B.Cu") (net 1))
 (segment (start 149.679733 105.25125) (end 143.805983 111.125) (width 0.25) (layer "B.Cu") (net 1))
 (segment (start 145.91375 41.275) (end 149.38375 44.745) (width 0.25) (layer "B.Cu") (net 1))
 (segment (start 143.805983 111.125) (end 105.56875 111.125) (width 0.25) (layer "B.Cu") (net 1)))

